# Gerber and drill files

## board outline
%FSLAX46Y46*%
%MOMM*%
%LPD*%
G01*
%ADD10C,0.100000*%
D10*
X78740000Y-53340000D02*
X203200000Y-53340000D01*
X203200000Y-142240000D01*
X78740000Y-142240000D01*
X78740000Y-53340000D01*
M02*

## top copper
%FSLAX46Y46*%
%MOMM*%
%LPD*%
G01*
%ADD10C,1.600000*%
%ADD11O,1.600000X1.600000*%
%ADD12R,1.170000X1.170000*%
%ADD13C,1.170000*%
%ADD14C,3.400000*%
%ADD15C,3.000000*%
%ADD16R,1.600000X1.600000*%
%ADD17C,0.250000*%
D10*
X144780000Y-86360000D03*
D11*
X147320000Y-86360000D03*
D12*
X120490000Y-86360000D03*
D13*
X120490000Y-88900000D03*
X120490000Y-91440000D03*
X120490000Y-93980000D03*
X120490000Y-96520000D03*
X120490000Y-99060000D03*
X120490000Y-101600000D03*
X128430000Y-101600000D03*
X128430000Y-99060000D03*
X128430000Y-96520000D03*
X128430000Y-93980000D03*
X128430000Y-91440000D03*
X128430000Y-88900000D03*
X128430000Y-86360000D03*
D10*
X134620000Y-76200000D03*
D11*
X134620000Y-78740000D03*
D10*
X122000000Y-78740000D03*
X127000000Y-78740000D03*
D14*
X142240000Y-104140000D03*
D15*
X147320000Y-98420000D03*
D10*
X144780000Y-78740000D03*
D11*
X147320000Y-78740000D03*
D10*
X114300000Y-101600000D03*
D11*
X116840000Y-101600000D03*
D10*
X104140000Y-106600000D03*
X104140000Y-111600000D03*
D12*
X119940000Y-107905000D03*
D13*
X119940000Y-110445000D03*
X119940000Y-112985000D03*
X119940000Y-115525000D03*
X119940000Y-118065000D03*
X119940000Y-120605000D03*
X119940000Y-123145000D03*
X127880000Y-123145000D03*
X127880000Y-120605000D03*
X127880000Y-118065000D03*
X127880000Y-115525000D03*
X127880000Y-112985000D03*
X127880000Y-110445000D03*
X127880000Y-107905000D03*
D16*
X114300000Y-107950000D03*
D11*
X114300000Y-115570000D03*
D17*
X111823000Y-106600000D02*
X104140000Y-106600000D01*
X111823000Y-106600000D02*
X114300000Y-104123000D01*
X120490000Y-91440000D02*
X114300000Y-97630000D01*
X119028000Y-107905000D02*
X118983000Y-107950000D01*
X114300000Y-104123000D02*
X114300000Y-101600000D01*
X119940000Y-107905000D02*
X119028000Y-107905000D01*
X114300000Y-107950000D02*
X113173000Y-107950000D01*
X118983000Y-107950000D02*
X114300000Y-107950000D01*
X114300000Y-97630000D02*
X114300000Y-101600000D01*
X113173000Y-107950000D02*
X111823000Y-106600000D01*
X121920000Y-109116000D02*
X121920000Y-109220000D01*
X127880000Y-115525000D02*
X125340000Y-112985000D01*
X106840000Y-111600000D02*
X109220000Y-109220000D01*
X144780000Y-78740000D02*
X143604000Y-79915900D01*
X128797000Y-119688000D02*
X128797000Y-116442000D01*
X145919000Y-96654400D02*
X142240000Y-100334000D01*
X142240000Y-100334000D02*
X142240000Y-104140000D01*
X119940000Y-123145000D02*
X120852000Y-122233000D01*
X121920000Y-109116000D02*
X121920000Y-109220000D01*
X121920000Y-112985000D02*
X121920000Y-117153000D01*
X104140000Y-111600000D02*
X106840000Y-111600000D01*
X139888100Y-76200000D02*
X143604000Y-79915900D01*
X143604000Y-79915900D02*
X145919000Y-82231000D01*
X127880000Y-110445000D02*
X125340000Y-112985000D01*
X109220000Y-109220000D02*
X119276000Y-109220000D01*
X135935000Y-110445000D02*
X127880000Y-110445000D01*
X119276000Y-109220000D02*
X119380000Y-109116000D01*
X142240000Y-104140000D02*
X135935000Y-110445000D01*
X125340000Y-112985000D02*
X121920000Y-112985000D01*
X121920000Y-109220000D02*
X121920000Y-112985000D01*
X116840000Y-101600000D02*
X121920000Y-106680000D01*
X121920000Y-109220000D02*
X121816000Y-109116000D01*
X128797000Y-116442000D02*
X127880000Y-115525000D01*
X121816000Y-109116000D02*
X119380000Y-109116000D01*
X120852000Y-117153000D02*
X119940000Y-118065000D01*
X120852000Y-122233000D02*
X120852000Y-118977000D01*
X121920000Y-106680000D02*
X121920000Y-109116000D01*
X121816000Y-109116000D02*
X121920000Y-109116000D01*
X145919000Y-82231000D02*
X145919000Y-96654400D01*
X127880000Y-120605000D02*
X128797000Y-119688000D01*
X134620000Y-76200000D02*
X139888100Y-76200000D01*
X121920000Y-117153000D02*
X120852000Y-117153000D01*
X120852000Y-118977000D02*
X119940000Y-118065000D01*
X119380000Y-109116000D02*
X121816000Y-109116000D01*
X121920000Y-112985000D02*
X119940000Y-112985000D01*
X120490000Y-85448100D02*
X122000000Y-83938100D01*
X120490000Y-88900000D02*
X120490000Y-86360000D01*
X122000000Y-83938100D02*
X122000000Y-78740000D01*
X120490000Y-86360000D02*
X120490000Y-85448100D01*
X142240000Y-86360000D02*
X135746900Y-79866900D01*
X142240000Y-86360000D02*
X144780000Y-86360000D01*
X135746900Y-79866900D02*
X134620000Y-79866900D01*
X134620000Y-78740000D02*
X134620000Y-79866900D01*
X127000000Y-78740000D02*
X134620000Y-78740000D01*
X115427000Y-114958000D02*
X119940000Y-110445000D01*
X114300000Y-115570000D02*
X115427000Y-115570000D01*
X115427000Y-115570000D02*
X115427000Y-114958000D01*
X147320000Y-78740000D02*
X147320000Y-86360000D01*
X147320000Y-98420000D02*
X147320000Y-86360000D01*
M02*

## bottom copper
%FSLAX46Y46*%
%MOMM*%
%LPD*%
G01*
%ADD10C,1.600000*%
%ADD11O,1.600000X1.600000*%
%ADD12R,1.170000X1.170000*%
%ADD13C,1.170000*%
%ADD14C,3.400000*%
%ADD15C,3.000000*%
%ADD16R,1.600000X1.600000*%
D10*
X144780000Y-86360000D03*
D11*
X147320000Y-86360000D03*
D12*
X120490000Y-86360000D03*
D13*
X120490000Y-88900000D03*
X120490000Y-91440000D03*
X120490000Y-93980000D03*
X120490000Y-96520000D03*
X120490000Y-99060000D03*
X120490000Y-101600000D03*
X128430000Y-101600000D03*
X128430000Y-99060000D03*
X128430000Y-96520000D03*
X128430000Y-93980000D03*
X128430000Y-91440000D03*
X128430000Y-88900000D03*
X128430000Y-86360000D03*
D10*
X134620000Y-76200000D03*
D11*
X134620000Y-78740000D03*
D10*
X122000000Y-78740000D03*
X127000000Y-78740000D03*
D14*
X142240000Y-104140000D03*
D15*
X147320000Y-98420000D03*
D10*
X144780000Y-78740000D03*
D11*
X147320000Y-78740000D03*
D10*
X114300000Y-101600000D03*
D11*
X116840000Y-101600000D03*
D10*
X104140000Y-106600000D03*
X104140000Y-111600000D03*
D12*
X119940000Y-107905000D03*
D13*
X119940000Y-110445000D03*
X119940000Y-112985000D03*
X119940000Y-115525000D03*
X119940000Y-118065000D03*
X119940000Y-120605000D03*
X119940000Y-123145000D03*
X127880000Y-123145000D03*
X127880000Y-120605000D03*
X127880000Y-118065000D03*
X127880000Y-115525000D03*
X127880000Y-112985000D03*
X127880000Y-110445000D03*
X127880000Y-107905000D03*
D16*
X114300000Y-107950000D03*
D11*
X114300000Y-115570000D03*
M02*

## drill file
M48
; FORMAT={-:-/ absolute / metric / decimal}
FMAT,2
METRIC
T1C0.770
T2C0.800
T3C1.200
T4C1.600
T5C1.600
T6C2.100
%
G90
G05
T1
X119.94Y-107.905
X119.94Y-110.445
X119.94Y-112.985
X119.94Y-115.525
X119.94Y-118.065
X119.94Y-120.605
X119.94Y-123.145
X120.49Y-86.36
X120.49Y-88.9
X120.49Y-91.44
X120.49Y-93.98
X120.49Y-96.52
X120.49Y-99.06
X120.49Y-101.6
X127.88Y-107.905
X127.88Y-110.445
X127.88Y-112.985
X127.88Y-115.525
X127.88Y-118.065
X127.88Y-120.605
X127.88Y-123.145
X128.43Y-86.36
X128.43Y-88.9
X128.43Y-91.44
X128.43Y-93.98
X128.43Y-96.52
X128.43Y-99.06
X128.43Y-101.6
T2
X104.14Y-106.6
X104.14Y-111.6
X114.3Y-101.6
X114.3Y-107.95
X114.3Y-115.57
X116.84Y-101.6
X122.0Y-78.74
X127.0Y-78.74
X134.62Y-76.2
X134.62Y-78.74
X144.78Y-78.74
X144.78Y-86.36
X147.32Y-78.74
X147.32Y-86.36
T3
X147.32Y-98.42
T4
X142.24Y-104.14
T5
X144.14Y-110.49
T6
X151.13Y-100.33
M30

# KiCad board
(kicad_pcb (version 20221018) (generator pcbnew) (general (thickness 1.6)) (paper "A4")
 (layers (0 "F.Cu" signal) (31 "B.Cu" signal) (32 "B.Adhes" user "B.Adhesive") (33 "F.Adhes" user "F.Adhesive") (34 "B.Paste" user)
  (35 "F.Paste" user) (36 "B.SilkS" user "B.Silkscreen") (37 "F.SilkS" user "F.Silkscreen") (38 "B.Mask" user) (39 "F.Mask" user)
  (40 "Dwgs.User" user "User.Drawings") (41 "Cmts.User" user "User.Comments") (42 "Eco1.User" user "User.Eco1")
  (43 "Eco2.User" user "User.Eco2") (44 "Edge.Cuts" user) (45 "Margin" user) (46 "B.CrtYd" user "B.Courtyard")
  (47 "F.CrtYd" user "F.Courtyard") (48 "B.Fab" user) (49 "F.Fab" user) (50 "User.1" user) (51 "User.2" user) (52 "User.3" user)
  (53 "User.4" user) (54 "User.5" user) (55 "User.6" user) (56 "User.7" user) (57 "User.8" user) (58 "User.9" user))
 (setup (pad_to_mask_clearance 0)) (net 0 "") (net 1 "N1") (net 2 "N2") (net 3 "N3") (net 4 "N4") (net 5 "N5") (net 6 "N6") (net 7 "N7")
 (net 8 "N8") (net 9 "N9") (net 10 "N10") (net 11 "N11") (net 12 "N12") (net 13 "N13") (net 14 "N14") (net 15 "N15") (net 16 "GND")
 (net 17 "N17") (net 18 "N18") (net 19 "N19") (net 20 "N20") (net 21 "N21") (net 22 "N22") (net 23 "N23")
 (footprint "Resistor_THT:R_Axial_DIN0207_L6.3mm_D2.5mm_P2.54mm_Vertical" (layer "F.Cu") (at 144.78 86.36)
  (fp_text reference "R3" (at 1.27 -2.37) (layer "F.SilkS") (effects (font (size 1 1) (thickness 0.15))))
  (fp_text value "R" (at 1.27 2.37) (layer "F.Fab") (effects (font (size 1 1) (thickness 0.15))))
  (pad "1" thru_hole circle (at 0 0) (size 1.6 1.6) (drill 0.8) (layers "*.Cu" "*.Mask") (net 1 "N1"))
  (pad "2" thru_hole oval (at 2.54 0) (size 1.6 1.6) (drill 0.8) (layers "*.Cu" "*.Mask") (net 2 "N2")))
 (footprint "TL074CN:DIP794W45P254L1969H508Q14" (layer "F.Cu") (at 124.46 93.98)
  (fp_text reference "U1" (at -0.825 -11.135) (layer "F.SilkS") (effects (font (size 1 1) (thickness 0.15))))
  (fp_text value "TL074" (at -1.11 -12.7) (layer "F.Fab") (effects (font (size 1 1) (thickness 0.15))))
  (pad "1" thru_hole rect (at -3.97 -7.62) (size 1.17 1.17) (drill 0.77) (layers "*.Cu" "*.Mask") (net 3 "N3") (solder_mask_margin 0.102))
  (pad "2" thru_hole circle (at -3.97 -5.08) (size 1.17 1.17) (drill 0.77) (layers "*.Cu" "*.Mask") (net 3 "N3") (solder_mask_margin 0.102))
  (pad "3" thru_hole circle (at -3.97 -2.54) (size 1.17 1.17) (drill 0.77) (layers "*.Cu" "*.Mask") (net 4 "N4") (solder_mask_margin 0.102))
  (pad "4" thru_hole circle (at -3.97 0) (size 1.17 1.17) (drill 0.77) (layers "*.Cu" "*.Mask") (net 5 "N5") (solder_mask_margin 0.102))
  (pad "5" thru_hole circle (at -3.97 2.54) (size 1.17 1.17) (drill 0.77) (layers "*.Cu" "*.Mask") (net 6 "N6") (solder_mask_margin 0.102))
  (pad "6" thru_hole circle (at -3.97 5.08) (size 1.17 1.17) (drill 0.77) (layers "*.Cu" "*.Mask") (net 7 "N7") (solder_mask_margin 0.102))
  (pad "7" thru_hole circle (at -3.97 7.62) (size 1.17 1.17) (drill 0.77) (layers "*.Cu" "*.Mask") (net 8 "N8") (solder_mask_margin 0.102))
  (pad "8" thru_hole circle (at 3.97 7.62) (size 1.17 1.17) (drill 0.77) (layers "*.Cu" "*.Mask") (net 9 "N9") (solder_mask_margin 0.102))
  (pad "9" thru_hole circle (at 3.97 5.08) (size 1.17 1.17) (drill 0.77) (layers "*.Cu" "*.Mask") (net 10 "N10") (solder_mask_margin 0.102))
  (pad "10" thru_hole circle (at 3.97 2.54) (size 1.17 1.17) (drill 0.77) (layers "*.Cu" "*.Mask") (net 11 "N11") (solder_mask_margin 0.102))
  (pad "11" thru_hole circle (at 3.97 0) (size 1.17 1.17) (drill 0.77) (layers "*.Cu" "*.Mask") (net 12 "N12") (solder_mask_margin 0.102))
  (pad "12" thru_hole circle (at 3.97 -2.54) (size 1.17 1.17) (drill 0.77) (layers "*.Cu" "*.Mask") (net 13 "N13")
   (solder_mask_margin 0.102))
  (pad "13" thru_hole circle (at 3.97 -5.08) (size 1.17 1.17) (drill 0.77) (layers "*.Cu" "*.Mask") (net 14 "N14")
   (solder_mask_margin 0.102))
  (pad "14" thru_hole circle (at 3.97 -7.62) (size 1.17 1.17) (drill 0.77) (layers "*.Cu" "*.Mask") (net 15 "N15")
   (solder_mask_margin 0.102)))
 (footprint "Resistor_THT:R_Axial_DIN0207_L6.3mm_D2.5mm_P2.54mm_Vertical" (layer "F.Cu") (at 134.62 76.2 -90)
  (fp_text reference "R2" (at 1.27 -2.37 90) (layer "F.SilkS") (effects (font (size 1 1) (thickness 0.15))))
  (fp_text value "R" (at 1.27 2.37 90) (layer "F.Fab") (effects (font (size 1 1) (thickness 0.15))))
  (pad "1" thru_hole circle (at 0 0 270) (size 1.6 1.6) (drill 0.8) (layers "*.Cu" "*.Mask") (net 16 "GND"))
  (pad "2" thru_hole oval (at 2.54 0 270) (size 1.6 1.6) (drill 0.8) (layers "*.Cu" "*.Mask") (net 1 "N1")))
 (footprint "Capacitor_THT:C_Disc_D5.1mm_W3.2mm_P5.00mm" (layer "F.Cu") (at 122 78.74)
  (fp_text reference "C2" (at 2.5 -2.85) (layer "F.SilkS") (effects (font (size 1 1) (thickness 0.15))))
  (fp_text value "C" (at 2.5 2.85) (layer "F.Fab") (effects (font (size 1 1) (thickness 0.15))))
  (pad "1" thru_hole circle (at 0 0) (size 1.6 1.6) (drill 0.8) (layers "*.Cu" "*.Mask") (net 3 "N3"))
  (pad "2" thru_hole circle (at 5 0) (size 1.6 1.6) (drill 0.8) (layers "*.Cu" "*.Mask") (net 1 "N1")))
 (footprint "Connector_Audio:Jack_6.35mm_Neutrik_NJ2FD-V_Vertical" (layer "F.Cu") (at 147.32 98.42)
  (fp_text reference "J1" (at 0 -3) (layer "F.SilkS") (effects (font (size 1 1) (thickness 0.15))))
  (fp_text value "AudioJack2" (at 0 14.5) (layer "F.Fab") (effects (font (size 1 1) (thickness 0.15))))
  (pad "" np_thru_hole circle (at -3.18 12.07 180) (size 1.6 1.6) (drill 1.6) (layers "*.Cu" "*.Mask"))
  (pad "" np_thru_hole circle (at 3.81 1.91 180) (size 2.1 2.1) (drill 2.1) (layers "*.Cu" "*.Mask"))
  (pad "S" thru_hole circle (at -5.08 5.72 180) (size 3.4 3.4) (drill 1.6) (layers "*.Cu" "*.Mask") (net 16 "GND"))
  (pad "T" thru_hole circle (at 0 0 180) (size 3 3) (drill 1.2) (layers "*.Cu" "*.Mask") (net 2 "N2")))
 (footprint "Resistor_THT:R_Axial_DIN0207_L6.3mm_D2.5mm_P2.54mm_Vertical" (layer "F.Cu") (at 144.78 78.74)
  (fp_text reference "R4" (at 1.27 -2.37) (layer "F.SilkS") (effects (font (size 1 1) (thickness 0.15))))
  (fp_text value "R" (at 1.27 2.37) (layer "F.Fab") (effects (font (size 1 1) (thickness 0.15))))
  (pad "1" thru_hole circle (at 0 0) (size 1.6 1.6) (drill 0.8) (layers "*.Cu" "*.Mask") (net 16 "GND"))
  (pad "2" thru_hole oval (at 2.54 0) (size 1.6 1.6) (drill 0.8) (layers "*.Cu" "*.Mask") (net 2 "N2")))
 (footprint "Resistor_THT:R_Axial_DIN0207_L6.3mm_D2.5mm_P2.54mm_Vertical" (layer "F.Cu") (at 114.3 101.6)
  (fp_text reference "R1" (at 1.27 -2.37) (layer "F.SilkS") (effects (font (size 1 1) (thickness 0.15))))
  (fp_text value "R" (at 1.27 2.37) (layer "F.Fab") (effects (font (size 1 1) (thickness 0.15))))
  (pad "1" thru_hole circle (at 0 0) (size 1.6 1.6) (drill 0.8) (layers "*.Cu" "*.Mask") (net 4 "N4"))
  (pad "2" thru_hole oval (at 2.54 0) (size 1.6 1.6) (drill 0.8) (layers "*.Cu" "*.Mask") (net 16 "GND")))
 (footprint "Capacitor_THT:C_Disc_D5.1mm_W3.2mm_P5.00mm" (layer "F.Cu") (at 104.14 106.6 -90)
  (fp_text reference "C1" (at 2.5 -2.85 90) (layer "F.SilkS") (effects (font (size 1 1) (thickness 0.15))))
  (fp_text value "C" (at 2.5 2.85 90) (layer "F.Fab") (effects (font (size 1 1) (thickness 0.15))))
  (pad "1" thru_hole circle (at 0 0 270) (size 1.6 1.6) (drill 0.8) (layers "*.Cu" "*.Mask") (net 4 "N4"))
  (pad "2" thru_hole circle (at 5 0 270) (size 1.6 1.6) (drill 0.8) (layers "*.Cu" "*.Mask") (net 16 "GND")))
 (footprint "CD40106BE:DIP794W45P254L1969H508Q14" (layer "F.Cu") (at 123.91 115.525)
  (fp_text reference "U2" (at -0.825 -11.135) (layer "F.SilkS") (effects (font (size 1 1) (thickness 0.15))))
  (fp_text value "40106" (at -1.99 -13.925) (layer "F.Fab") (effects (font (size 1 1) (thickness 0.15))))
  (pad "1" thru_hole rect (at -3.97 -7.62) (size 1.17 1.17) (drill 0.77) (layers "*.Cu" "*.Mask") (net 4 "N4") (solder_mask_margin 0.102))
  (pad "2" thru_hole circle (at -3.97 -5.08) (size 1.17 1.17) (drill 0.77) (layers "*.Cu" "*.Mask") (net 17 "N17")
   (solder_mask_margin 0.102))
  (pad "3" thru_hole circle (at -3.97 -2.54) (size 1.17 1.17) (drill 0.77) (layers "*.Cu" "*.Mask") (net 16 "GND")
   (solder_mask_margin 0.102))
  (pad "4" thru_hole circle (at -3.97 0) (size 1.17 1.17) (drill 0.77) (layers "*.Cu" "*.Mask") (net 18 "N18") (solder_mask_margin 0.102))
  (pad "5" thru_hole circle (at -3.97 2.54) (size 1.17 1.17) (drill 0.77) (layers "*.Cu" "*.Mask") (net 16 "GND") (solder_mask_margin 0.102))
  (pad "6" thru_hole circle (at -3.97 5.08) (size 1.17 1.17) (drill 0.77) (layers "*.Cu" "*.Mask") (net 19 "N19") (solder_mask_margin 0.102))
  (pad "7" thru_hole circle (at -3.97 7.62) (size 1.17 1.17) (drill 0.77) (layers "*.Cu" "*.Mask") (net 16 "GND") (solder_mask_margin 0.102))
  (pad "8" thru_hole circle (at 3.97 7.62) (size 1.17 1.17) (drill 0.77) (layers "*.Cu" "*.Mask") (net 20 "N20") (solder_mask_margin 0.102))
  (pad "9" thru_hole circle (at 3.97 5.08) (size 1.17 1.17) (drill 0.77) (layers "*.Cu" "*.Mask") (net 16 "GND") (solder_mask_margin 0.102))
  (pad "10" thru_hole circle (at 3.97 2.54) (size 1.17 1.17) (drill 0.77) (layers "*.Cu" "*.Mask") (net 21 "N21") (solder_mask_margin 0.102))
  (pad "11" thru_hole circle (at 3.97 0) (size 1.17 1.17) (drill 0.77) (layers "*.Cu" "*.Mask") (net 16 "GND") (solder_mask_margin 0.102))
  (pad "12" thru_hole circle (at 3.97 -2.54) (size 1.17 1.17) (drill 0.77) (layers "*.Cu" "*.Mask") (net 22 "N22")
   (solder_mask_margin 0.102))
  (pad "13" thru_hole circle (at 3.97 -5.08) (size 1.17 1.17) (drill 0.77) (layers "*.Cu" "*.Mask") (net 16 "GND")
   (solder_mask_margin 0.102))
  (pad "14" thru_hole circle (at 3.97 -7.62) (size 1.17 1.17) (drill 0.77) (layers "*.Cu" "*.Mask") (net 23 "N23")
   (solder_mask_margin 0.102)))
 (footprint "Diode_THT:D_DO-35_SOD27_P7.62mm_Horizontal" (layer "F.Cu") (at 114.3 107.95 -90)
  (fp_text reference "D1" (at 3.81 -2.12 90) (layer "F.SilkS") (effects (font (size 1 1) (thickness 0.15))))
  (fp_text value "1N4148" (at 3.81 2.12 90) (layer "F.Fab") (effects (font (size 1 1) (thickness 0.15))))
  (pad "1" thru_hole rect (at 0 0 270) (size 1.6 1.6) (drill 0.8) (layers "*.Cu" "*.Mask") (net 4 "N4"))
  (pad "2" thru_hole oval (at 7.62 0 270) (size 1.6 1.6) (drill 0.8) (layers "*.Cu" "*.Mask") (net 17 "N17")))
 (gr_rect (start 78.74 53.34) (end 203.2 142.24) (stroke (width 0.1) (type default)) (fill none) (layer "Edge.Cuts"))
 (segment (start 111.823 106.6) (end 104.14 106.6) (width 0.25) (layer "F.Cu") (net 4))
 (segment (start 111.823 106.6) (end 114.3 104.123) (width 0.25) (layer "F.Cu") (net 4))
 (segment (start 120.49 91.44) (end 114.3 97.63) (width 0.25) (layer "F.Cu") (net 4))
 (segment (start 119.028 107.905) (end 118.983 107.95) (width 0.25) (layer "F.Cu") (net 4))
 (segment (start 114.3 104.123) (end 114.3 101.6) (width 0.25) (layer "F.Cu") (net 4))
 (segment (start 119.94 107.905) (end 119.028 107.905) (width 0.25) (layer "F.Cu") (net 4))
 (segment (start 114.3 107.95) (end 113.173 107.95) (width 0.25) (layer "F.Cu") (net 4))
 (segment (start 118.983 107.95) (end 114.3 107.95) (width 0.25) (layer "F.Cu") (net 4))
 (segment (start 114.3 97.63) (end 114.3 101.6) (width 0.25) (layer "F.Cu") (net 4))
 (segment (start 113.173 107.95) (end 111.823 106.6) (width 0.25) (layer "F.Cu") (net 4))
 (segment (start 121.92 109.116) (end 121.92 109.22) (width 0.25) (layer "F.Cu") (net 16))
 (segment (start 127.88 115.525) (end 125.34 112.985) (width 0.25) (layer "F.Cu") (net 16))
 (segment (start 106.84 111.6) (end 109.22 109.22) (width 0.25) (layer "F.Cu") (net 16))
 (segment (start 144.78 78.74) (end 143.604 79.9159) (width 0.25) (layer "F.Cu") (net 16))
 (segment (start 128.797 119.688) (end 128.797 116.442) (width 0.25) (layer "F.Cu") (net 16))
 (segment (start 145.919 96.6544) (end 142.24 100.334) (width 0.25) (layer "F.Cu") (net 16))
 (segment (start 142.24 100.334) (end 142.24 104.14) (width 0.25) (layer "F.Cu") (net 16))
 (segment (start 119.94 123.145) (end 120.852 122.233) (width 0.25) (layer "F.Cu") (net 16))
 (segment (start 121.92 109.116) (end 121.92 109.22) (width 0.25) (layer "F.Cu") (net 16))
 (segment (start 121.92 112.985) (end 121.92 117.153) (width 0.25) (layer "F.Cu") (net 16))
 (segment (start 104.14 111.6) (end 106.84 111.6) (width 0.25) (layer "F.Cu") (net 16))
 (segment (start 139.8881 76.2) (end 143.604 79.9159) (width 0.25) (layer "F.Cu") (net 16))
 (segment (start 143.604 79.9159) (end 145.919 82.231) (width 0.25) (layer "F.Cu") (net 16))
 (segment (start 127.88 110.445) (end 125.34 112.985) (width 0.25) (layer "F.Cu") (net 16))
 (segment (start 109.22 109.22) (end 119.276 109.22) (width 0.25) (layer "F.Cu") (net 16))
 (segment (start 135.935 110.445) (end 127.88 110.445) (width 0.25) (layer "F.Cu") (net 16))
 (segment (start 119.276 109.22) (end 119.38 109.116) (width 0.25) (layer "F.Cu") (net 16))
 (segment (start 142.24 104.14) (end 135.935 110.445) (width 0.25) (layer "F.Cu") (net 16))
 (segment (start 125.34 112.985) (end 121.92 112.985) (width 0.25) (layer "F.Cu") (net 16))
 (segment (start 121.92 109.22) (end 121.92 112.985) (width 0.25) (layer "F.Cu") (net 16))
 (segment (start 116.84 101.6) (end 121.92 106.68) (width 0.25) (layer "F.Cu") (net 16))
 (segment (start 121.92 109.22) (end 121.816 109.116) (width 0.25) (layer "F.Cu") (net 16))
 (segment (start 128.797 116.442) (end 127.88 115.525) (width 0.25) (layer "F.Cu") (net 16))
 (segment (start 121.816 109.116) (end 119.38 109.116) (width 0.25) (layer "F.Cu") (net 16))
 (segment (start 120.852 117.153) (end 119.94 118.065) (width 0.25) (layer "F.Cu") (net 16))
 (segment (start 120.852 122.233) (end 120.852 118.977) (width 0.25) (layer "F.Cu") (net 16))
 (segment (start 121.92 106.68) (end 121.92 109.116) (width 0.25) (layer "F.Cu") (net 16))
 (segment (start 121.816 109.116) (end 121.92 109.116) (width 0.25) (layer "F.Cu") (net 16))
 (segment (start 145.919 82.231) (end 145.919 96.6544) (width 0.25) (layer "F.Cu") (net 16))
 (segment (start 127.88 120.605) (end 128.797 119.688) (width 0.25) (layer "F.Cu") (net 16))
 (segment (start 134.62 76.2) (end 139.8881 76.2) (width 0.25) (layer "F.Cu") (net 16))
 (segment (start 121.92 117.153) (end 120.852 117.153) (width 0.25) (layer "F.Cu") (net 16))
 (segment (start 120.852 118.977) (end 119.94 118.065) (width 0.25) (layer "F.Cu") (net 16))
 (segment (start 119.38 109.116) (end 121.816 109.116) (width 0.25) (layer "F.Cu") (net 16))
 (segment (start 121.92 112.985) (end 119.94 112.985) (width 0.25) (layer "F.Cu") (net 16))
 (segment (start 120.49 85.4481) (end 122 83.9381) (width 0.25) (layer "F.Cu") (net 3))
 (segment (start 120.49 88.9) (end 120.49 86.36) (width 0.25) (layer "F.Cu") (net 3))
 (segment (start 122 83.9381) (end 122 78.74) (width 0.25) (layer "F.Cu") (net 3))
 (segment (start 120.49 86.36) (end 120.49 85.4481) (width 0.25) (layer "F.Cu") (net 3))
 (segment (start 142.24 86.36) (end 135.7469 79.8669) (width 0.25) (layer "F.Cu") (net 1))
 (segment (start 142.24 86.36) (end 144.78 86.36) (width 0.25) (layer "F.Cu") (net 1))
 (segment (start 135.7469 79.8669) (end 134.62 79.8669) (width 0.25) (layer "F.Cu") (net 1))
 (segment (start 134.62 78.74) (end 134.62 79.8669) (width 0.25) (layer "F.Cu") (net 1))
 (segment (start 127 78.74) (end 134.62 78.74) (width 0.25) (layer "F.Cu") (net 1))
 (segment (start 115.427 114.958) (end 119.94 110.445) (width 0.25) (layer "F.Cu") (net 17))
 (segment (start 114.3 115.57) (end 115.427 115.57) (width 0.25) (layer "F.Cu") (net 17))
 (segment (start 115.427 115.57) (end 115.427 114.958) (width 0.25) (layer "F.Cu") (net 17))
 (segment (start 147.32 78.74) (end 147.32 86.36) (width 0.25) (layer "F.Cu") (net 2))
 (segment (start 147.32 98.42) (end 147.32 86.36) (width 0.25) (layer "F.Cu") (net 2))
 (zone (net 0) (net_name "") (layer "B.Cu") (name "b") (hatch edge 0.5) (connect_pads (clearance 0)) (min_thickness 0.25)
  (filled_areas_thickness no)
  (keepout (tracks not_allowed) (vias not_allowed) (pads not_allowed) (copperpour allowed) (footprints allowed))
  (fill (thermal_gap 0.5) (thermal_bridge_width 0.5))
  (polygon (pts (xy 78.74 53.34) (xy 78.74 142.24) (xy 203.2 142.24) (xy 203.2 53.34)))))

